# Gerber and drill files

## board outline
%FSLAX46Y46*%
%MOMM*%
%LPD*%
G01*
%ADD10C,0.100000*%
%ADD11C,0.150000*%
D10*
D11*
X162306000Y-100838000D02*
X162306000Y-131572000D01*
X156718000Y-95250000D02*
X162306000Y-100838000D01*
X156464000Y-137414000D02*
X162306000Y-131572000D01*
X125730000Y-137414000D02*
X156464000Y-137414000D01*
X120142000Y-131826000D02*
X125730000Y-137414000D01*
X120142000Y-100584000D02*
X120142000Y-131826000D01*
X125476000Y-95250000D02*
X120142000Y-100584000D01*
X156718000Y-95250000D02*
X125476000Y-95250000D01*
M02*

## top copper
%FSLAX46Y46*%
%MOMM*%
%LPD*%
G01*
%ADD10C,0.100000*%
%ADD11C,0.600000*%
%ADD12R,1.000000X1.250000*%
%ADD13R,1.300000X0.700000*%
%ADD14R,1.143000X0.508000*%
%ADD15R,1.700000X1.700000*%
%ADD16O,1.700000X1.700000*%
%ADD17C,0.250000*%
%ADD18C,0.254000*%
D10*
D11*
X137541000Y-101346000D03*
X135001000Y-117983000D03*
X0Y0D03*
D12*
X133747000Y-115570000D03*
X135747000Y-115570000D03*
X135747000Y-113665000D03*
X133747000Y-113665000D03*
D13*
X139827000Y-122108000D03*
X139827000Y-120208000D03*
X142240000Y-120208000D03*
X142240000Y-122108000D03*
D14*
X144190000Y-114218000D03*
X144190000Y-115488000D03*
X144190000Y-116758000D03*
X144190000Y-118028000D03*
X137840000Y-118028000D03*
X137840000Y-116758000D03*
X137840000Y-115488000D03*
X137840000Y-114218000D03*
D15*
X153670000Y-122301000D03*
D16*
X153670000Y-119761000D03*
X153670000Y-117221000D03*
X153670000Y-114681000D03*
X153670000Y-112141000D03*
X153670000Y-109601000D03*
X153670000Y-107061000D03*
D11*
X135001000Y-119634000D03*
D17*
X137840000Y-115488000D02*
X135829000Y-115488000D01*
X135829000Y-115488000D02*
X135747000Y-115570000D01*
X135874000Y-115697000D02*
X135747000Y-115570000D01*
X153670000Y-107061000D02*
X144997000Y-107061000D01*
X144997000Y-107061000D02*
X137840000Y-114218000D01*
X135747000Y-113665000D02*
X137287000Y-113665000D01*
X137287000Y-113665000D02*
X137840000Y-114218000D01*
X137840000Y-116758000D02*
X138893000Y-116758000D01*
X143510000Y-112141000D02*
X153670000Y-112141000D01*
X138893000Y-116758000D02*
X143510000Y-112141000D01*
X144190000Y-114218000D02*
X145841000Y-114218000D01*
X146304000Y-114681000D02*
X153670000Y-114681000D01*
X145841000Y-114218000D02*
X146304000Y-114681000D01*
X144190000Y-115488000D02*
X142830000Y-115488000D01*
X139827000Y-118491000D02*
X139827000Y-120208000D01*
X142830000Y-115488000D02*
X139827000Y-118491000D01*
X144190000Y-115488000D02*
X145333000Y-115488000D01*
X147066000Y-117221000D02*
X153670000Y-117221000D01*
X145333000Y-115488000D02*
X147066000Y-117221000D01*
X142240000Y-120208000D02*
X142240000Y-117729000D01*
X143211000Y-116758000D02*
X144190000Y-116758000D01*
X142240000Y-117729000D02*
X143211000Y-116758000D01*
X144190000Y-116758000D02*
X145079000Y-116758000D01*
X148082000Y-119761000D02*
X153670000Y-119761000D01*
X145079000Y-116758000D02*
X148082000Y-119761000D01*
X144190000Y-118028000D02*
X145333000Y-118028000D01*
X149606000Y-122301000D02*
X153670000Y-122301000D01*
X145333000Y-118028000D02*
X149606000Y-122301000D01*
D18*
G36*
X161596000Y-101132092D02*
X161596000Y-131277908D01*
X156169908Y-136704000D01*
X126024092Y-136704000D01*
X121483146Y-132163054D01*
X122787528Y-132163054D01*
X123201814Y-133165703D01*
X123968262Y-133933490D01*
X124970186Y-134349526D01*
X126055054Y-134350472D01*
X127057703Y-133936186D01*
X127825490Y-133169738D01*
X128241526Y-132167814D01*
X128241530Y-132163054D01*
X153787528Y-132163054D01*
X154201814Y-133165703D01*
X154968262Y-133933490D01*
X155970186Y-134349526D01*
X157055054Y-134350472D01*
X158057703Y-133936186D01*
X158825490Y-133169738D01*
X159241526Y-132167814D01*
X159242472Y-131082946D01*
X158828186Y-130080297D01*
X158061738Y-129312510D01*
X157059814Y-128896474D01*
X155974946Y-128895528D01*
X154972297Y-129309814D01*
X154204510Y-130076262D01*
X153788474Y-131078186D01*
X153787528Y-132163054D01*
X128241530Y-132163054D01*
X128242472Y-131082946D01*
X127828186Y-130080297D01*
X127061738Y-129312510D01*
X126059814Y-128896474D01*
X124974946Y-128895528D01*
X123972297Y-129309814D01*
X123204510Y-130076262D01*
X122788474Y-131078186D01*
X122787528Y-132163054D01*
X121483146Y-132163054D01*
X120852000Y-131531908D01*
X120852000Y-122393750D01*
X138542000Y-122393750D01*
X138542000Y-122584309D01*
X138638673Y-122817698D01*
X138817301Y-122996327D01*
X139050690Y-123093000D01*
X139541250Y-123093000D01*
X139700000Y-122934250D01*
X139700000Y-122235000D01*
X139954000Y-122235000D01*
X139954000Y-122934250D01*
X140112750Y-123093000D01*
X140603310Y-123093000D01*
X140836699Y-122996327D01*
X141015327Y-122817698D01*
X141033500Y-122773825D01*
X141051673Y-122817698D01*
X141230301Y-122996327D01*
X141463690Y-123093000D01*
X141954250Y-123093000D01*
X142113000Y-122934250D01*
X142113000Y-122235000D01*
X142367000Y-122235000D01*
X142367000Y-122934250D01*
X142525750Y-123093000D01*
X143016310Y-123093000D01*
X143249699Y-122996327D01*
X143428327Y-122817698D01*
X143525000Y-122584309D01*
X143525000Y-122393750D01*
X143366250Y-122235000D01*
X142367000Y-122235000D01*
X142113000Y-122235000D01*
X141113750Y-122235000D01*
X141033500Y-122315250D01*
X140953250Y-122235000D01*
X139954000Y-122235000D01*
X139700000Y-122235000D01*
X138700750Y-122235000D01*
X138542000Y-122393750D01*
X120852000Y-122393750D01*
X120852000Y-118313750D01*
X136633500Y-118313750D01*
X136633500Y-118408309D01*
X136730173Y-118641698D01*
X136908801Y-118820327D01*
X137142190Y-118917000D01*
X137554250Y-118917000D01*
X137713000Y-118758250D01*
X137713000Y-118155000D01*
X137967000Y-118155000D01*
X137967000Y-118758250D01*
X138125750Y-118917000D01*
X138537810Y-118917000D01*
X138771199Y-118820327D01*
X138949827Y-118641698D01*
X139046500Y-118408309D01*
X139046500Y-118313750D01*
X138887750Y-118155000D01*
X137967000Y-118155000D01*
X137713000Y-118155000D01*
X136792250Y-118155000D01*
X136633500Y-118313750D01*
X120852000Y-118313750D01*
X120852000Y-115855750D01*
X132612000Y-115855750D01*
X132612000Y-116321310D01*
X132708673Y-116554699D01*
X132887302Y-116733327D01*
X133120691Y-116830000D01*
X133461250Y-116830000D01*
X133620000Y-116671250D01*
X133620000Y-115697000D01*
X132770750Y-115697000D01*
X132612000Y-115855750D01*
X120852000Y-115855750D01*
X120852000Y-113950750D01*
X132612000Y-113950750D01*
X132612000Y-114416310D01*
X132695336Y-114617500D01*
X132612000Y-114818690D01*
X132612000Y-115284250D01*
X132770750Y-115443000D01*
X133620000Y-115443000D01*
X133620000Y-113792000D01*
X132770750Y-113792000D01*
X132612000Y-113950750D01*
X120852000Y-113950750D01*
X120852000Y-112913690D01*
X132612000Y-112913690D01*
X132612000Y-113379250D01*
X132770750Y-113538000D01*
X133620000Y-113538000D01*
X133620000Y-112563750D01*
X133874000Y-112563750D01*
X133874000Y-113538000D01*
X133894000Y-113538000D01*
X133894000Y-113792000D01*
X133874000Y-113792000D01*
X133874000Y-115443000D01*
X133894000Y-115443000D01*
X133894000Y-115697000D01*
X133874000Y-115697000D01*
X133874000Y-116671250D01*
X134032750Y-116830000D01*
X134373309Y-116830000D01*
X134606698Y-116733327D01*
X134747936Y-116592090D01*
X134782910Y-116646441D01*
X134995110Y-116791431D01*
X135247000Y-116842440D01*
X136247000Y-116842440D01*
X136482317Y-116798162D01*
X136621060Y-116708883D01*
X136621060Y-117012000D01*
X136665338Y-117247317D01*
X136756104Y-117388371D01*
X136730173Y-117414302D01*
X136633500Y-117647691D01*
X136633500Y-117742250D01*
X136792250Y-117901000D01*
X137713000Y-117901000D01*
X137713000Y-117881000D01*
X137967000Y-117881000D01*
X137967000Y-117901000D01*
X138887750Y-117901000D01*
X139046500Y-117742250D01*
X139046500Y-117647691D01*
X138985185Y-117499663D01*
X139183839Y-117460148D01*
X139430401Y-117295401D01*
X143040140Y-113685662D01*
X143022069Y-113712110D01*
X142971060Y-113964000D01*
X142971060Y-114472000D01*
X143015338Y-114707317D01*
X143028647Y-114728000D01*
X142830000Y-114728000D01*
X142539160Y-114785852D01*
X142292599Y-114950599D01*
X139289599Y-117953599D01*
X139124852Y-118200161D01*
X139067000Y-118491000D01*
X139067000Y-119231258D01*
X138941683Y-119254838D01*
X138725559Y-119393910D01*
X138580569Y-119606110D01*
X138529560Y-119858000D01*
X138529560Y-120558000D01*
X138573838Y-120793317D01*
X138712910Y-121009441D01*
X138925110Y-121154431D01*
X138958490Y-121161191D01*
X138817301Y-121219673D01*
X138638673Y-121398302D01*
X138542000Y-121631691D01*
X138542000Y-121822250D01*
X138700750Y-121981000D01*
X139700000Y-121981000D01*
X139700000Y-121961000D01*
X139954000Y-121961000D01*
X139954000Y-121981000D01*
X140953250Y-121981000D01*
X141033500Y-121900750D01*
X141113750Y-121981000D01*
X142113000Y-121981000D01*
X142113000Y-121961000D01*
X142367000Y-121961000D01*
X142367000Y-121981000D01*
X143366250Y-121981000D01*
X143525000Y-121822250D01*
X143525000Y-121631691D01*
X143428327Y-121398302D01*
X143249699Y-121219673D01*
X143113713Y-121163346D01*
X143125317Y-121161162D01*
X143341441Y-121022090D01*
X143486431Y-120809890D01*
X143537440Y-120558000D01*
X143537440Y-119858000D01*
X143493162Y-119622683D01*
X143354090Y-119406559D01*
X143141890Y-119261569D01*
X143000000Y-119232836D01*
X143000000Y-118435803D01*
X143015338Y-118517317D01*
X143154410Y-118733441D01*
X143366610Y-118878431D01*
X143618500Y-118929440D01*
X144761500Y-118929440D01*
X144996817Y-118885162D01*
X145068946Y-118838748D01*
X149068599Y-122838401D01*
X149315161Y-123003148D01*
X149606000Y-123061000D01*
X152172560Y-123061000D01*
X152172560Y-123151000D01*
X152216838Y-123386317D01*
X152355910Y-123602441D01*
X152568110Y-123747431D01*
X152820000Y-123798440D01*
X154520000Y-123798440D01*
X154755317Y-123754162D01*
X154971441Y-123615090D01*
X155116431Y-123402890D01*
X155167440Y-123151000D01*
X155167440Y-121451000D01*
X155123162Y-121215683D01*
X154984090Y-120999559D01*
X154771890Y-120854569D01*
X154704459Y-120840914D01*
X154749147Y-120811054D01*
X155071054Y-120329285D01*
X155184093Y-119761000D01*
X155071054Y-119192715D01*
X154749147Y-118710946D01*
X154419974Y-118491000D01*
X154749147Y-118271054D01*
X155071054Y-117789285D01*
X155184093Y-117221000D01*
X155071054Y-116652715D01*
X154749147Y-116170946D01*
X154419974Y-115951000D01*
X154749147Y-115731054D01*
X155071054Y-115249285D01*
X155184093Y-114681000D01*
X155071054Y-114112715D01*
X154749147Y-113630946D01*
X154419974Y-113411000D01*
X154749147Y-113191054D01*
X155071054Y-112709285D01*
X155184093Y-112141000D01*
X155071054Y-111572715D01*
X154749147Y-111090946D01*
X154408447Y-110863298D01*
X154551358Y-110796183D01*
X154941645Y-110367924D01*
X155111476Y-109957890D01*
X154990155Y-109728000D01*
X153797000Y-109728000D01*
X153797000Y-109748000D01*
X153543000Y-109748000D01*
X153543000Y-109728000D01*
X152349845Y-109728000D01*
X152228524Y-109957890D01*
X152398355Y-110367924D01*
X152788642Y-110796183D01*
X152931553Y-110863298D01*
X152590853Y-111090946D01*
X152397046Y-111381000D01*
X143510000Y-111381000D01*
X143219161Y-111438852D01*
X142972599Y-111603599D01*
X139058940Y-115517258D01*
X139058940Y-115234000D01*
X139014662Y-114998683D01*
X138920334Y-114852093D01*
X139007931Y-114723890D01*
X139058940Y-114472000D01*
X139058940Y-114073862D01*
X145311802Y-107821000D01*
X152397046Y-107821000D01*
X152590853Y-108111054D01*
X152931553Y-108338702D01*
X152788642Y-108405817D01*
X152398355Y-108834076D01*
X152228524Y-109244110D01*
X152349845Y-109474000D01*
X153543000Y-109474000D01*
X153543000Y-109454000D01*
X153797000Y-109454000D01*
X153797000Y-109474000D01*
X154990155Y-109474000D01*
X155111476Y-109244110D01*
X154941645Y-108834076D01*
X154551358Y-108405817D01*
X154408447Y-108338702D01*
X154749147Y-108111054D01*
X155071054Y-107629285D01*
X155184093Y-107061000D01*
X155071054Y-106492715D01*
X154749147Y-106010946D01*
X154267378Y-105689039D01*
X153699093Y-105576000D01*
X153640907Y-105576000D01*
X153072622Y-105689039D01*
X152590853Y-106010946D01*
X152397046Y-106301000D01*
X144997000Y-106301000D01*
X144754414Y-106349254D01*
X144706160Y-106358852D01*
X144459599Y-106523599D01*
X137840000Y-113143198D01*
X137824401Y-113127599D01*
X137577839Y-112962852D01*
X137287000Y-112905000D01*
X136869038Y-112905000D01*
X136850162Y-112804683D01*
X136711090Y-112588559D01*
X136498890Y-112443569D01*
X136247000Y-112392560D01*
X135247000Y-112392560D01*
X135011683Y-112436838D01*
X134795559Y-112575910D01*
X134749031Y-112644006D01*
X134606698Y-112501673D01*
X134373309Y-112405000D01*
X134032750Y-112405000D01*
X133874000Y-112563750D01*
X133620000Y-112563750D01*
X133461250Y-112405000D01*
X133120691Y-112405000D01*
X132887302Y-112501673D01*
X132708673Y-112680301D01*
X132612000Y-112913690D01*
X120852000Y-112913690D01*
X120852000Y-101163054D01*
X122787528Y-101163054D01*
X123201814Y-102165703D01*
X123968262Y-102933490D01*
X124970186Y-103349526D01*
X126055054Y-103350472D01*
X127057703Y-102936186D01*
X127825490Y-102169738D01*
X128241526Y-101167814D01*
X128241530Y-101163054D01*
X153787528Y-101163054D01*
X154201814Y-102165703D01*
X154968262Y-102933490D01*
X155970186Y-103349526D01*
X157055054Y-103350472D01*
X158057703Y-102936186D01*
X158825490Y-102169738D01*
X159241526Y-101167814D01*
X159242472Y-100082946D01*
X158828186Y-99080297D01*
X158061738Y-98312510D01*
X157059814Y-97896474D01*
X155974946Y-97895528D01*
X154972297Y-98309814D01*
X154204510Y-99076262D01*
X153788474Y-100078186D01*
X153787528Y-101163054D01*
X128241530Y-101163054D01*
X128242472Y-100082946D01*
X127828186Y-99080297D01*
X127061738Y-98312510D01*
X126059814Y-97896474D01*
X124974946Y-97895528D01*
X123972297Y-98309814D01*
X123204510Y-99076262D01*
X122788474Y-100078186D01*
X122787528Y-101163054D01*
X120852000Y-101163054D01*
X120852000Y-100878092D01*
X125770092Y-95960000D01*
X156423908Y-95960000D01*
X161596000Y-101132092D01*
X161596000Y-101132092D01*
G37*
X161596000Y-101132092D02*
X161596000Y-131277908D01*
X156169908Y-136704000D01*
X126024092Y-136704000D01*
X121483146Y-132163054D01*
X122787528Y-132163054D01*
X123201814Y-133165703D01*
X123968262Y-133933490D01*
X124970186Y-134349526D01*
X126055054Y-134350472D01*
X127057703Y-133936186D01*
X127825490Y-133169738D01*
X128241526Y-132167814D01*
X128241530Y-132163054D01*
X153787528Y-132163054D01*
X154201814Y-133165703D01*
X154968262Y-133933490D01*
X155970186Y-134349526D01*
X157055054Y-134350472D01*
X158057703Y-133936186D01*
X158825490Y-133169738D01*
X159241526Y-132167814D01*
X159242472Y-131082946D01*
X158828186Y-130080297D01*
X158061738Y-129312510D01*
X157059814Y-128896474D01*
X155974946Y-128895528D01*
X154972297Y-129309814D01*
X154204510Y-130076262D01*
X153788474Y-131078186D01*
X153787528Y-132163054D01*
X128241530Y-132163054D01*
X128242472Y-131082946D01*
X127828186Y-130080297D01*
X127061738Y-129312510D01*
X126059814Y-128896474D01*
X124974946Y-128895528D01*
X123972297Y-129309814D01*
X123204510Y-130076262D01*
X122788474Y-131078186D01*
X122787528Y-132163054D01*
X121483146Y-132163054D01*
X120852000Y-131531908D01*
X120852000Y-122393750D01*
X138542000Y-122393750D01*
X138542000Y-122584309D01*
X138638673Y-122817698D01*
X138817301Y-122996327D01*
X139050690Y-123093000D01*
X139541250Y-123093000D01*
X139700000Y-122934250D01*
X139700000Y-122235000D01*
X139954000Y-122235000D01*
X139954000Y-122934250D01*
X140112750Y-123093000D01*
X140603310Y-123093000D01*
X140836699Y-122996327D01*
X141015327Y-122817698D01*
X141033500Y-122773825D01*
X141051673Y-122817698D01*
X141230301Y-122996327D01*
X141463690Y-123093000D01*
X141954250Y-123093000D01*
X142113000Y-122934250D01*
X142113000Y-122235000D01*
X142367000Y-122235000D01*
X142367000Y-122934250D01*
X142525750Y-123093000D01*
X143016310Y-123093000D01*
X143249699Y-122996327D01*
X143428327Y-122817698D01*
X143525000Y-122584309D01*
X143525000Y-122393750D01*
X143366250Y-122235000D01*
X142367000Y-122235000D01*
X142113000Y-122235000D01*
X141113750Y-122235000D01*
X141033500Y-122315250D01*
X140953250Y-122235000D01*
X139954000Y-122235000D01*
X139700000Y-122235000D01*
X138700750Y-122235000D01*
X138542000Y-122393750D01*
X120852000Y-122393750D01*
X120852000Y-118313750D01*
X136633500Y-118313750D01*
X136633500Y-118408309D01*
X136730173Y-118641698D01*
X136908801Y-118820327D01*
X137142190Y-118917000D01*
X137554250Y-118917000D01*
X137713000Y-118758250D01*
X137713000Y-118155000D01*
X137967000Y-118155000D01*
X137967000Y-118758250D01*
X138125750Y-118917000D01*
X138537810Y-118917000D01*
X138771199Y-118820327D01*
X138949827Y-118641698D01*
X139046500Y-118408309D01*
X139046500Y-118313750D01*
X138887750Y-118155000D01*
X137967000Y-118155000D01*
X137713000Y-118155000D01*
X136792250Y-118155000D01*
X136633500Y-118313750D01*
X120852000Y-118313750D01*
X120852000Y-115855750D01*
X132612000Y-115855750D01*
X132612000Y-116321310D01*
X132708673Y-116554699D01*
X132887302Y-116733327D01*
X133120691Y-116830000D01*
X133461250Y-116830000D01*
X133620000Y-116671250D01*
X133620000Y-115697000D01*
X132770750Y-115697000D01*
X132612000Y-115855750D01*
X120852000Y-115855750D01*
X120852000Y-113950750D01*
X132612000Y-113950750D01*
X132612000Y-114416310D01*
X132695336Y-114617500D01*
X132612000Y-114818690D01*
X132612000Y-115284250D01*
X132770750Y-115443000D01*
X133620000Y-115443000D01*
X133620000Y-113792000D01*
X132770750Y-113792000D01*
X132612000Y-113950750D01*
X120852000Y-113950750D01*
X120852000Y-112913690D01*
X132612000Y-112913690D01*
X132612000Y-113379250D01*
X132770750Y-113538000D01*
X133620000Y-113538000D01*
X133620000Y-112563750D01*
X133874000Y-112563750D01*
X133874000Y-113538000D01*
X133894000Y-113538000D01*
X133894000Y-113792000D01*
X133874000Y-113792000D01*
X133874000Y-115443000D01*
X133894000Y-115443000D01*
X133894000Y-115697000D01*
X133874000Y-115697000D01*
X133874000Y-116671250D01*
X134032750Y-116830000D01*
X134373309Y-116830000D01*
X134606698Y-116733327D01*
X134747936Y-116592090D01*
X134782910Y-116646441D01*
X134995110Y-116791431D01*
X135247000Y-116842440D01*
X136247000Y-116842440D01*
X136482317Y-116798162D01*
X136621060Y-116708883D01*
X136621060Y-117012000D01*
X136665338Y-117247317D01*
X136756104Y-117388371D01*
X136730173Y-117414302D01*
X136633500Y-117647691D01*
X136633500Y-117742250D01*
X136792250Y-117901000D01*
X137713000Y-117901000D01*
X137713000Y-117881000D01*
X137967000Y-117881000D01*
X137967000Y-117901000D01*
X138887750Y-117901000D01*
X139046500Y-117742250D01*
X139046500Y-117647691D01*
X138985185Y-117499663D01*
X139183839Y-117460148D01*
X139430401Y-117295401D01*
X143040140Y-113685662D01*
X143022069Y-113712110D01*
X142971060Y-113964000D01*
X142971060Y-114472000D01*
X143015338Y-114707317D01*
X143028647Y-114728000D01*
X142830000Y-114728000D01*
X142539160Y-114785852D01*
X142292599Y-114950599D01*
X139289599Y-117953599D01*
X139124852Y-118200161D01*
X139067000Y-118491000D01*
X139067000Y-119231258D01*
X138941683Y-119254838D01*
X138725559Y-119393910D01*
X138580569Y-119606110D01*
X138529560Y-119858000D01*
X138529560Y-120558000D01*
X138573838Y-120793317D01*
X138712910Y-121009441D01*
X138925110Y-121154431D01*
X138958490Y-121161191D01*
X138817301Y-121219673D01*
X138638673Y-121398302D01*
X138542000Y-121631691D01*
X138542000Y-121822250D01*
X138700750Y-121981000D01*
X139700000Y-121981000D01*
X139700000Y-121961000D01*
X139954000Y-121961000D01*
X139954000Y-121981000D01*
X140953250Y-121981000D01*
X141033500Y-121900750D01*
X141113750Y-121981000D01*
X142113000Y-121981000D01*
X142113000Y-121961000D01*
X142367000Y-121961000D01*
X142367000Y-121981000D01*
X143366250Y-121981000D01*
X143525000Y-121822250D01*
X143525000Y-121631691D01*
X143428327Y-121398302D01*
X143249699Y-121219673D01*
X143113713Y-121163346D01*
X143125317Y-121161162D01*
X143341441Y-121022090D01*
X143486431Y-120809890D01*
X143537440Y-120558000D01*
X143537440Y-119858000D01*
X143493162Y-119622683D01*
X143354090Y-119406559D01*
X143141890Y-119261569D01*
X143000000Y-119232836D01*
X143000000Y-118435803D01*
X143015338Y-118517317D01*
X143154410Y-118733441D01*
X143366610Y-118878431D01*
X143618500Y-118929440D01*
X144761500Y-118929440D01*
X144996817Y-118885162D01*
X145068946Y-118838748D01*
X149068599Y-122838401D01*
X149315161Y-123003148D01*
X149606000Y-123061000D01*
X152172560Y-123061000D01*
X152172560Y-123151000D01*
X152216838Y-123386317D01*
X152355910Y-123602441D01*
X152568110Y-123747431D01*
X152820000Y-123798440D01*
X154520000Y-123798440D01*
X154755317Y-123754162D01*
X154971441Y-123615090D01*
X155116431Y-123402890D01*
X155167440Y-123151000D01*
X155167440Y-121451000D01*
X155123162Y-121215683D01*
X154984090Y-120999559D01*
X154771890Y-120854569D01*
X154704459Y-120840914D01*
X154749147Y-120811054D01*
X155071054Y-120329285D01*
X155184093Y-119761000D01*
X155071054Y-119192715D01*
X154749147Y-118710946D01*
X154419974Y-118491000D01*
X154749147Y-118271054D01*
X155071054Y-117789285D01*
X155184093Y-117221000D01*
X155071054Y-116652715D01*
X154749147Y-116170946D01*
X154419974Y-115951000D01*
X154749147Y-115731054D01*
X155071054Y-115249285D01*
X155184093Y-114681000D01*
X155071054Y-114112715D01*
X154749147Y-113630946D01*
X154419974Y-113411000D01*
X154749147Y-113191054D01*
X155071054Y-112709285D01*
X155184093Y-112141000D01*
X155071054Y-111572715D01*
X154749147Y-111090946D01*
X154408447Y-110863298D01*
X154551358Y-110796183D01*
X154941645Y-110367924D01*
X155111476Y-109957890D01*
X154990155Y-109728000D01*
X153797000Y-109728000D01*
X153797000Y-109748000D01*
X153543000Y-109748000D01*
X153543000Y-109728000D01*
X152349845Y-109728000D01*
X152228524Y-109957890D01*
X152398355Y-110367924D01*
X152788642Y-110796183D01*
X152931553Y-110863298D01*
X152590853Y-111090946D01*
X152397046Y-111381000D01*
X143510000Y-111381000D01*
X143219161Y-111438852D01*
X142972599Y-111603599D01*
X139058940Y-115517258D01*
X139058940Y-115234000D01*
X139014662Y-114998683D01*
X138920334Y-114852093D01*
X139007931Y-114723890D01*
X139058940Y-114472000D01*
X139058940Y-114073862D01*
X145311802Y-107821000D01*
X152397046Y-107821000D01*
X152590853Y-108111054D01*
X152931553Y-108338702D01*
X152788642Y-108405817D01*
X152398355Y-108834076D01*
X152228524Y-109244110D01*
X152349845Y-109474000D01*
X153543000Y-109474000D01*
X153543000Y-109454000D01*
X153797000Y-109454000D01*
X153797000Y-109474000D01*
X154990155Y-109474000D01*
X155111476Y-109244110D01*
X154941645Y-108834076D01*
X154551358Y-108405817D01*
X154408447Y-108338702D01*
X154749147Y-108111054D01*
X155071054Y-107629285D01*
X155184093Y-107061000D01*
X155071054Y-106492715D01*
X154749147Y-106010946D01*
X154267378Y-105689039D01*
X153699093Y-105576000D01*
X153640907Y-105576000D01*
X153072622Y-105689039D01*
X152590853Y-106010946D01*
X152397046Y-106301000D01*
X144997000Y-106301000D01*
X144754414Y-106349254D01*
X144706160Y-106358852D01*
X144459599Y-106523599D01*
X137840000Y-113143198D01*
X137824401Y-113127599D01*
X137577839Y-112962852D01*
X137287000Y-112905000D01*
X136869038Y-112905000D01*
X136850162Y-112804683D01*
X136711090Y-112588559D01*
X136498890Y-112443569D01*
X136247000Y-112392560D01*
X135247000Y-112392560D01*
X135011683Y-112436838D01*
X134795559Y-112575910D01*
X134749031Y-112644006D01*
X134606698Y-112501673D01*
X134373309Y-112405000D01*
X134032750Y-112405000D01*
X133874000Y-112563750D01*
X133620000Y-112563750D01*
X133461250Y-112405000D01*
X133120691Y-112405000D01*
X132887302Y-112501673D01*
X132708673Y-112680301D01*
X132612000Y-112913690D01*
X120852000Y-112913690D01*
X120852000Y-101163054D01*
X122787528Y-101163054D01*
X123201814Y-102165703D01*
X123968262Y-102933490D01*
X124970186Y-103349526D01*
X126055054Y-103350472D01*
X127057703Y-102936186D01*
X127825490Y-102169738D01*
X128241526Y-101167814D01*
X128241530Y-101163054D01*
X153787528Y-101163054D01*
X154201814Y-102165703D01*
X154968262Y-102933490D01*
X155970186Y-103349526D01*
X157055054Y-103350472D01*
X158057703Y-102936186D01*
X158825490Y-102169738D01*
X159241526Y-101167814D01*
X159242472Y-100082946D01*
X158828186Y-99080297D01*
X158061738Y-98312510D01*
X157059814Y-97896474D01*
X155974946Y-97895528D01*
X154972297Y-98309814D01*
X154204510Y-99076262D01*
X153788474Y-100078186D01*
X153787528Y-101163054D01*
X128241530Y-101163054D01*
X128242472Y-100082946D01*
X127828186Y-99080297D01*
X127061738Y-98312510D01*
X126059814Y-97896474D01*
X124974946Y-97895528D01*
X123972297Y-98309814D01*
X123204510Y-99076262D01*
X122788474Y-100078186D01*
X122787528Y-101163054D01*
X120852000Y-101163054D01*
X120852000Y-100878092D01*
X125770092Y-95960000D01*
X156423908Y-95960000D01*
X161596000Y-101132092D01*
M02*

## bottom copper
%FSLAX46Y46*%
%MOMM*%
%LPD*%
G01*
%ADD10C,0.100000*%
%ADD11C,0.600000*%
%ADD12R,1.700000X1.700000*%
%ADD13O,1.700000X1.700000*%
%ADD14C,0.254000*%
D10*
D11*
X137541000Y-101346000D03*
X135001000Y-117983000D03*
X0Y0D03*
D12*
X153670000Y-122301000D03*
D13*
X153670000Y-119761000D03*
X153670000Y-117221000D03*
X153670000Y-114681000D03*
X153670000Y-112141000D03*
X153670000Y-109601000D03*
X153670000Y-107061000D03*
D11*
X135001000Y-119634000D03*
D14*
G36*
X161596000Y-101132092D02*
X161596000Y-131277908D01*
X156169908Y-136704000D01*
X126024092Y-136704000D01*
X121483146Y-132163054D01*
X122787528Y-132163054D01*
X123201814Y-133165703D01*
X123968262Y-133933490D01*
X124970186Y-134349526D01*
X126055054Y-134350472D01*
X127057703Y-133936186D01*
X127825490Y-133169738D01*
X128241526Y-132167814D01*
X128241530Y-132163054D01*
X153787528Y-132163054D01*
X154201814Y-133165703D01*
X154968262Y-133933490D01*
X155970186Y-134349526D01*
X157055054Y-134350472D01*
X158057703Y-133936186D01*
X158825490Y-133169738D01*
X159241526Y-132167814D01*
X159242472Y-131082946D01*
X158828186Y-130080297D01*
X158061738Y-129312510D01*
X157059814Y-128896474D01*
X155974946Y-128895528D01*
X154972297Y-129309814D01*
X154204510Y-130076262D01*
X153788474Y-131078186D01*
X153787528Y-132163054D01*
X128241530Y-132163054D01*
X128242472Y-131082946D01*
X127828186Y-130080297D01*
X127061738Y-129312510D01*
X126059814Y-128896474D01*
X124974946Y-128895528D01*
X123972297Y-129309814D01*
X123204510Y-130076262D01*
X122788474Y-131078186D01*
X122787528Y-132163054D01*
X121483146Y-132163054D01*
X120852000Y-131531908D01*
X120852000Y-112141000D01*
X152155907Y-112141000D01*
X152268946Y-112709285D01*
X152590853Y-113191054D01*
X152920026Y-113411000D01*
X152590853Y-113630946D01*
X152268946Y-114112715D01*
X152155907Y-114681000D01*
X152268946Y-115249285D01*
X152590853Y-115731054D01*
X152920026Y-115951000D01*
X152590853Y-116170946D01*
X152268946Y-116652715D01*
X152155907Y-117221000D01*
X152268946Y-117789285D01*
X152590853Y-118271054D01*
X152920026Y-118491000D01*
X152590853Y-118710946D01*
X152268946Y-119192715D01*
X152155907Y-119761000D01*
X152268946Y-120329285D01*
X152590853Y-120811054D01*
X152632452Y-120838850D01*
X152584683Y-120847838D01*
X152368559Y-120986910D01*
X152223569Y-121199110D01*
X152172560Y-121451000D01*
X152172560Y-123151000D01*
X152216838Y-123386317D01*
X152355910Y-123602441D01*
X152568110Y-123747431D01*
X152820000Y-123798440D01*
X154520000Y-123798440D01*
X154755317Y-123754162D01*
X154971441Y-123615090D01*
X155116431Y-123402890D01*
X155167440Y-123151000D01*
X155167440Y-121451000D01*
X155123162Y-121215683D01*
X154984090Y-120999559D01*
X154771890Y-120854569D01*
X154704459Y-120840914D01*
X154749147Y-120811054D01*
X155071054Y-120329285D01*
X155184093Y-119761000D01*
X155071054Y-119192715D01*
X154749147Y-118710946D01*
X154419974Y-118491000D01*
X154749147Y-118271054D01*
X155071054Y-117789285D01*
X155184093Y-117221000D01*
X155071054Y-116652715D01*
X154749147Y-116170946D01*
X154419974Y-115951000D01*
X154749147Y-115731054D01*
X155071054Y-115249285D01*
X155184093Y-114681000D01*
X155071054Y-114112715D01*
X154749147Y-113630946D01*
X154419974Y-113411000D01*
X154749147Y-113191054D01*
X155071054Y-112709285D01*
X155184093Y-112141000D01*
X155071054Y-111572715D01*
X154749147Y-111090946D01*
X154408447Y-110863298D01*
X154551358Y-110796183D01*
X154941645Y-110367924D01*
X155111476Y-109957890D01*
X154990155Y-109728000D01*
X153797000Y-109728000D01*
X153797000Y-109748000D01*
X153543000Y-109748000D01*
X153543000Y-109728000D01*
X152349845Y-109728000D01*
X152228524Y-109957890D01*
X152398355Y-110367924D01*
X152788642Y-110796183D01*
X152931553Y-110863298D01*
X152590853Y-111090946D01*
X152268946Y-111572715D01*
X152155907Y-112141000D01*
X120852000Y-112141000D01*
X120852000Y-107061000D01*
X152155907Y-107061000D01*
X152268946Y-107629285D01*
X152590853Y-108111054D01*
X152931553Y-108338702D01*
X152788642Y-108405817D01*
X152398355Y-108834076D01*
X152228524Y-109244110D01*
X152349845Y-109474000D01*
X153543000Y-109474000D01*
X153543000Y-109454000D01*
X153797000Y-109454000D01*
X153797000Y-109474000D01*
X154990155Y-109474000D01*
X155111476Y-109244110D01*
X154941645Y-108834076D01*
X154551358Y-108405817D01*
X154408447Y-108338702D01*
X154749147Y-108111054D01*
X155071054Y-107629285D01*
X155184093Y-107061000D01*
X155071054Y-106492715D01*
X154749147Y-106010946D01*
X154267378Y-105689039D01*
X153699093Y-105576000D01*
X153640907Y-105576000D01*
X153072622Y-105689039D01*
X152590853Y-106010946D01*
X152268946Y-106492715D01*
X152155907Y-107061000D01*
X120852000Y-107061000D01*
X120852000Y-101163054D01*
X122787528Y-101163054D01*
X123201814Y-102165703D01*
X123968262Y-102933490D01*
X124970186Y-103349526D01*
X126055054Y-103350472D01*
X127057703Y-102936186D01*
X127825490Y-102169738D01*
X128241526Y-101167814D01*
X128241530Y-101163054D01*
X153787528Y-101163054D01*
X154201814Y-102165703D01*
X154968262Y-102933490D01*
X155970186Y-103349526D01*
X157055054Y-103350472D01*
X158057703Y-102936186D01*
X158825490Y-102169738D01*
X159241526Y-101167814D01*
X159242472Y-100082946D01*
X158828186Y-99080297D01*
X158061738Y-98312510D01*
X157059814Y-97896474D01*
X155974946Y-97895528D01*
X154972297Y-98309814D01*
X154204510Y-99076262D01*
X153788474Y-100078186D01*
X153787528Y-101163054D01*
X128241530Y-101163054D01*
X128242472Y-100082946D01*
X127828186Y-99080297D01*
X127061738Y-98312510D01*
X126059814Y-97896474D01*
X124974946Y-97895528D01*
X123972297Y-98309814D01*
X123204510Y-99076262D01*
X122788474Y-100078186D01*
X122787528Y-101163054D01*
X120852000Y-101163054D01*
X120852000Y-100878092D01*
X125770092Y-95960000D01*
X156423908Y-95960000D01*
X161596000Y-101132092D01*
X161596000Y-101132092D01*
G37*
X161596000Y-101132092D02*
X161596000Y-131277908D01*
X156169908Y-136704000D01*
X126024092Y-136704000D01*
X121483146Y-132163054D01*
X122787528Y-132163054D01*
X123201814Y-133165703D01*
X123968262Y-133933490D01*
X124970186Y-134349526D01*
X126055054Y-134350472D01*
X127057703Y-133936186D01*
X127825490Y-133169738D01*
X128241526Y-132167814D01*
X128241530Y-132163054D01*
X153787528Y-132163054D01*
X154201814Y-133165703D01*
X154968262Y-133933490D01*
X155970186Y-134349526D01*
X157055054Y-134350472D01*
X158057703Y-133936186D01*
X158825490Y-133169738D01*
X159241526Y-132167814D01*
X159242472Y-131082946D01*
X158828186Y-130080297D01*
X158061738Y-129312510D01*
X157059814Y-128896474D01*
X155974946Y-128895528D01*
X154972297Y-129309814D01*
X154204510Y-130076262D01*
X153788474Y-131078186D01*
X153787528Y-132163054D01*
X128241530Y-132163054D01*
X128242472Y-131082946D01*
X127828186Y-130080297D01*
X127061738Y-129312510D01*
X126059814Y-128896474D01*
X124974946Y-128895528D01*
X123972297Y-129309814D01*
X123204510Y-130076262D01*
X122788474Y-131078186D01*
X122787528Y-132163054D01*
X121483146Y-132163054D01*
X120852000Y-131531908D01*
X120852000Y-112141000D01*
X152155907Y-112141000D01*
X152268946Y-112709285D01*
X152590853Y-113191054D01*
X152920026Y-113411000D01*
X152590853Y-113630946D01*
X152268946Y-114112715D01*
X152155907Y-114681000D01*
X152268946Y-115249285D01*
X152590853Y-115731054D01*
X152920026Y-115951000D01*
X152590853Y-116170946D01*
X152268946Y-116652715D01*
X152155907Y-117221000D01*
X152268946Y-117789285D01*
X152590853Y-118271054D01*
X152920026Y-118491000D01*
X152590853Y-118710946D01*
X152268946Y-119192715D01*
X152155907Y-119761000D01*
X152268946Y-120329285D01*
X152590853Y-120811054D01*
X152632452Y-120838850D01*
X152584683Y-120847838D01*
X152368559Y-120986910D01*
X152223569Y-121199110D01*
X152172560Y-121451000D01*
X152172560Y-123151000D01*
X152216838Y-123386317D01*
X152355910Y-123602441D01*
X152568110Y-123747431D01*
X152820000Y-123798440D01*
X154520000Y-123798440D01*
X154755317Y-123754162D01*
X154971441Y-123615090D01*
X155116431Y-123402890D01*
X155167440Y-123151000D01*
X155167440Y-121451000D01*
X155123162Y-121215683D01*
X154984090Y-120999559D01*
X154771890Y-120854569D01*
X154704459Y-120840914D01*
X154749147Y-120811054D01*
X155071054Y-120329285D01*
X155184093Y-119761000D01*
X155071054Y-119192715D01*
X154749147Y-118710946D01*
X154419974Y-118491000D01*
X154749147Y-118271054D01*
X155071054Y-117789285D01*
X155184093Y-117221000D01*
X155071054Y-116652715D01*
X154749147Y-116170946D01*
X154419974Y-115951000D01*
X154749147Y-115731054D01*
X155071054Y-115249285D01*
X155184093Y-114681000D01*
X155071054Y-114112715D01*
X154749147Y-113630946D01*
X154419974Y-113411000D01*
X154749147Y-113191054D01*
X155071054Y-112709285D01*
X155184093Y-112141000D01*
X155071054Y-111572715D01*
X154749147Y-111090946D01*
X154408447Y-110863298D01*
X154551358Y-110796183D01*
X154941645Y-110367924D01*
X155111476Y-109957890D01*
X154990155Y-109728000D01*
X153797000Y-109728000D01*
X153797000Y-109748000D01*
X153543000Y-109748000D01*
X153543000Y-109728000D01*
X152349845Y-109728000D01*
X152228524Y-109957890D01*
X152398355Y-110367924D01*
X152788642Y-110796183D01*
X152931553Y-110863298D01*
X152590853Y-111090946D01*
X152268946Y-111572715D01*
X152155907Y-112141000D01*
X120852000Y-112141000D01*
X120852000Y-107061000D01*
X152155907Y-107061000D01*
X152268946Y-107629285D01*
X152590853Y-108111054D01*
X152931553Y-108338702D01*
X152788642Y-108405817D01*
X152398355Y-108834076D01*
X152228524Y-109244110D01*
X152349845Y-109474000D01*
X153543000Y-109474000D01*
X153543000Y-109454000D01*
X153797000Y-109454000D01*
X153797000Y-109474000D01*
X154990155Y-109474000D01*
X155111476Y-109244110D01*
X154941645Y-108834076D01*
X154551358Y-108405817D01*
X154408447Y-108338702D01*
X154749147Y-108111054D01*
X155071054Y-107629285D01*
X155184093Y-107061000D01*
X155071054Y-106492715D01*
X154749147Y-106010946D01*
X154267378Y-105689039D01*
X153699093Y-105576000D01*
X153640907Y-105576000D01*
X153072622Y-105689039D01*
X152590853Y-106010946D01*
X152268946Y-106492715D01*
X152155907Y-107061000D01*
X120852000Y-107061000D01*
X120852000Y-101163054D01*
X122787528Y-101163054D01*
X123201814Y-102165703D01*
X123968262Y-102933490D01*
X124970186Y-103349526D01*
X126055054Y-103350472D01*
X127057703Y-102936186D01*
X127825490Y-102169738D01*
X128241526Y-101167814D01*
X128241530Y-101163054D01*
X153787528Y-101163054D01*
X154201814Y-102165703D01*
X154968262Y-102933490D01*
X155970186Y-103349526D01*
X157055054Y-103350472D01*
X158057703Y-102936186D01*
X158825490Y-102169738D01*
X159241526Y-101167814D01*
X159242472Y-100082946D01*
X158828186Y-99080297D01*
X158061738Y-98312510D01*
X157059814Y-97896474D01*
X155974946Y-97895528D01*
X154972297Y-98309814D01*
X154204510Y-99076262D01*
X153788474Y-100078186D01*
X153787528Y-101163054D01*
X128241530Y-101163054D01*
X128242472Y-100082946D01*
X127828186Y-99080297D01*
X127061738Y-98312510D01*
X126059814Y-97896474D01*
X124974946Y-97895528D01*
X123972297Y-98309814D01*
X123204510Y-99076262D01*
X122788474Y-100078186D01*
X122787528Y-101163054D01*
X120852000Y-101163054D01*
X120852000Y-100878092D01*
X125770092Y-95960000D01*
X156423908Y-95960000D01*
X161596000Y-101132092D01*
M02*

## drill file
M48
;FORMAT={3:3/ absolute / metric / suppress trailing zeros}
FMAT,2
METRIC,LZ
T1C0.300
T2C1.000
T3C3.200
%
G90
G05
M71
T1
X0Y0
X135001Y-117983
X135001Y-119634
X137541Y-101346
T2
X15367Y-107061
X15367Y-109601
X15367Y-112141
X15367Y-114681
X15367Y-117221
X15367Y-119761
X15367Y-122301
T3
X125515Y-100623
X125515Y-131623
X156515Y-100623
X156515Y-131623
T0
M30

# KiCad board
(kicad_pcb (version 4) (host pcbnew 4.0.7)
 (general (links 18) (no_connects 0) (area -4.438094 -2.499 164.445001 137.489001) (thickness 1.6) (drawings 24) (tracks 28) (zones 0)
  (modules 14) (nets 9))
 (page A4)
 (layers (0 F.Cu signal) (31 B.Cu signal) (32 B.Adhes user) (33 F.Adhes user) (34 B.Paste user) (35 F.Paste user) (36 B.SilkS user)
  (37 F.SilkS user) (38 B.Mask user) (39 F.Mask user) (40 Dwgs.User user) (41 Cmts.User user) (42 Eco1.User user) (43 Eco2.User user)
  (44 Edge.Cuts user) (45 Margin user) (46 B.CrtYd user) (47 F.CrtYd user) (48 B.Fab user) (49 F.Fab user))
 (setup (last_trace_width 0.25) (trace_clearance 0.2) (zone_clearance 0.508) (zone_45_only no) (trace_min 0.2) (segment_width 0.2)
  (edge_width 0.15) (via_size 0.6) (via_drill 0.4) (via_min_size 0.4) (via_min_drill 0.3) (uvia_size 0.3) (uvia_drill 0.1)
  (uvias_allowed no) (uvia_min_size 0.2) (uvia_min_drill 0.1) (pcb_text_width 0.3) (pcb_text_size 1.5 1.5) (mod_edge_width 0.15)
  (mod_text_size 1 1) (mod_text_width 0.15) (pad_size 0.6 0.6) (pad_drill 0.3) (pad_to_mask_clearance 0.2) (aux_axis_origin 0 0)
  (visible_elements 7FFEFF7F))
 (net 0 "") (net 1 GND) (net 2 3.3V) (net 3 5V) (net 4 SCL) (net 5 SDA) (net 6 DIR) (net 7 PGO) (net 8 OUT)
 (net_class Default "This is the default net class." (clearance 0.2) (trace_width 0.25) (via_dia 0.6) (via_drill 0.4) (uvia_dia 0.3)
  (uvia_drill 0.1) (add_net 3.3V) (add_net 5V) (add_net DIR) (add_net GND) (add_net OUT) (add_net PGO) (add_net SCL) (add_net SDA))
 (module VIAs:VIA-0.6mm (layer F.Cu) (at 137.541 101.346)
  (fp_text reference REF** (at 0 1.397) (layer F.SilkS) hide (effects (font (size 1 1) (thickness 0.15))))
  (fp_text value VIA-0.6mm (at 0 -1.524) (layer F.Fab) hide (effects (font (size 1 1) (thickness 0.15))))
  (pad 1 thru_hole circle (at 0 0) (size 0.6 0.6) (drill 0.3) (layers *.Cu) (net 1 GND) (zone_connect 2)))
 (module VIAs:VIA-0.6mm (layer F.Cu) (at 135.001 117.983)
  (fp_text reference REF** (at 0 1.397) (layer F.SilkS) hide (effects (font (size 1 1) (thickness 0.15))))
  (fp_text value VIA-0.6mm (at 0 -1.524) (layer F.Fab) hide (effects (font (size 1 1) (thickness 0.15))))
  (pad 1 thru_hole circle (at 0 0) (size 0.6 0.6) (drill 0.3) (layers *.Cu) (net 1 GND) (zone_connect 2)))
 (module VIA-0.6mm (layer F.Cu) (at 0 0)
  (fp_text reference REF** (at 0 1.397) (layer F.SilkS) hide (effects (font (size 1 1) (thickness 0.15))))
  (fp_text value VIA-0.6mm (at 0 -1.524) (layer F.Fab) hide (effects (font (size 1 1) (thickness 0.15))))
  (pad 1 thru_hole circle (at 0 0) (size 0.6 0.6) (drill 0.3) (layers *.Cu) (zone_connect 2)))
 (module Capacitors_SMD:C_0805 (layer F.Cu) (at 134.747 115.57)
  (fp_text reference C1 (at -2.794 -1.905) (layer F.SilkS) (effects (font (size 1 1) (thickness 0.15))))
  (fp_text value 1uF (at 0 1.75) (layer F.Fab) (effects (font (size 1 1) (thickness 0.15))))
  (pad 1 smd rect (at -1 0) (size 1 1.25) (layers F.Cu F.Paste F.Mask) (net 1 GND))
  (pad 2 smd rect (at 1 0) (size 1 1.25) (layers F.Cu F.Paste F.Mask) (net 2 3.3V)))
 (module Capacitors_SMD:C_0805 (layer F.Cu) (at 134.747 113.665 180)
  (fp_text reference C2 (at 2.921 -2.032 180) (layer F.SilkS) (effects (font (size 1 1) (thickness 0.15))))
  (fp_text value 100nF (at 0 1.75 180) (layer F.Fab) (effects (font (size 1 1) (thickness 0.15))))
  (pad 1 smd rect (at -1 0 180) (size 1 1.25) (layers F.Cu F.Paste F.Mask) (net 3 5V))
  (pad 2 smd rect (at 1 0 180) (size 1 1.25) (layers F.Cu F.Paste F.Mask) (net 1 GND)))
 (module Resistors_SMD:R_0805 (layer F.Cu) (at 139.827 121.158 90)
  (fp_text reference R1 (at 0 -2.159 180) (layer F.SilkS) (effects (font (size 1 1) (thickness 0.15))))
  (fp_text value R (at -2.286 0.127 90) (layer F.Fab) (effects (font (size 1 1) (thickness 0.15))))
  (pad 1 smd rect (at -0.95 0 90) (size 0.7 1.3) (layers F.Cu F.Paste F.Mask) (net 1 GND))
  (pad 2 smd rect (at 0.95 0 90) (size 0.7 1.3) (layers F.Cu F.Paste F.Mask) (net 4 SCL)))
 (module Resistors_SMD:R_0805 (layer F.Cu) (at 142.24 121.158 270)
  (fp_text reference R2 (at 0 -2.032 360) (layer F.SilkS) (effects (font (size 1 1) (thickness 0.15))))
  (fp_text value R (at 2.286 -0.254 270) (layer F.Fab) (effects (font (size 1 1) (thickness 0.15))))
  (pad 1 smd rect (at -0.95 0 270) (size 0.7 1.3) (layers F.Cu F.Paste F.Mask) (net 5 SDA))
  (pad 2 smd rect (at 0.95 0 270) (size 0.7 1.3) (layers F.Cu F.Paste F.Mask) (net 1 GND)))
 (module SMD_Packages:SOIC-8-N (layer F.Cu) (at 141.015 116.123 270)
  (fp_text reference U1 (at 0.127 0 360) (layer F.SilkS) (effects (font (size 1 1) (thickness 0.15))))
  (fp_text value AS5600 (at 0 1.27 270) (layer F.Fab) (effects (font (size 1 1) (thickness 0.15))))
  (pad 8 smd rect (at -1.905 -3.175 270) (size 0.508 1.143) (layers F.Cu F.Paste F.Mask) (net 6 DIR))
  (pad 7 smd rect (at -0.635 -3.175 270) (size 0.508 1.143) (layers F.Cu F.Paste F.Mask) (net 4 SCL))
  (pad 6 smd rect (at 0.635 -3.175 270) (size 0.508 1.143) (layers F.Cu F.Paste F.Mask) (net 5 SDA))
  (pad 5 smd rect (at 1.905 -3.175 270) (size 0.508 1.143) (layers F.Cu F.Paste F.Mask) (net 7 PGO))
  (pad 4 smd rect (at 1.905 3.175 270) (size 0.508 1.143) (layers F.Cu F.Paste F.Mask) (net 1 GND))
  (pad 3 smd rect (at 0.635 3.175 270) (size 0.508 1.143) (layers F.Cu F.Paste F.Mask) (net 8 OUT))
  (pad 2 smd rect (at -0.635 3.175 270) (size 0.508 1.143) (layers F.Cu F.Paste F.Mask) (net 2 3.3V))
  (pad 1 smd rect (at -1.905 3.175 270) (size 0.508 1.143) (layers F.Cu F.Paste F.Mask) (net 3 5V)))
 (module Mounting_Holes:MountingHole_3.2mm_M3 (layer F.Cu) (at 125.515 100.623) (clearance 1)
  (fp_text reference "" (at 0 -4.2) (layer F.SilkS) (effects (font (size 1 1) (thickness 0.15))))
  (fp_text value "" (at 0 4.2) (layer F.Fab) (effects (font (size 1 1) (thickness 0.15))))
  (pad 1 np_thru_hole circle (at 0 0) (size 3.2 3.2) (drill 3.2) (layers *.Cu *.Mask)))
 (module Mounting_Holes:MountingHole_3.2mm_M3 (layer F.Cu) (at 156.515 100.623) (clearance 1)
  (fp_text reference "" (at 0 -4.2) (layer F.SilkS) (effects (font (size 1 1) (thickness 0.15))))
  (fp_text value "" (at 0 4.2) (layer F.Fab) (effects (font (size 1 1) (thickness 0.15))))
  (pad 1 np_thru_hole circle (at 0 0) (size 3.2 3.2) (drill 3.2) (layers *.Cu *.Mask)))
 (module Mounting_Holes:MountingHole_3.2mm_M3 (layer F.Cu) (at 125.515 131.623) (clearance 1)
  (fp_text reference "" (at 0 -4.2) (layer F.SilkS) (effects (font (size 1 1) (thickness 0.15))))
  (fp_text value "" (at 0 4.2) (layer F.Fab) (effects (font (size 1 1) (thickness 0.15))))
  (pad 1 np_thru_hole circle (at 0 0) (size 3.2 3.2) (drill 3.2) (layers *.Cu *.Mask)))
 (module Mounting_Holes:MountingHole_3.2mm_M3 (layer F.Cu) (at 156.515 131.623) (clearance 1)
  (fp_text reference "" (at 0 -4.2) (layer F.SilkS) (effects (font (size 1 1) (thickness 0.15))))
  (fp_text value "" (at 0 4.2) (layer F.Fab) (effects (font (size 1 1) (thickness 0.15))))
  (pad 1 np_thru_hole circle (at 0 0) (size 3.2 3.2) (drill 3.2) (layers *.Cu *.Mask)))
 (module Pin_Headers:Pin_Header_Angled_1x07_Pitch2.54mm (layer B.Cu) (at 153.67 122.301)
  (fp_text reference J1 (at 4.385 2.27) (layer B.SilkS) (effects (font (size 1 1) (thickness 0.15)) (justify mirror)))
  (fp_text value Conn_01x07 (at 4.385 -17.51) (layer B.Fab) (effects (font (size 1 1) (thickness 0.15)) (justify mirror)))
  (pad 1 thru_hole rect (at 0 0) (size 1.7 1.7) (drill 1) (layers *.Cu *.Mask) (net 7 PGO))
  (pad 2 thru_hole oval (at 0 -2.54) (size 1.7 1.7) (drill 1) (layers *.Cu *.Mask) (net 5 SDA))
  (pad 3 thru_hole oval (at 0 -5.08) (size 1.7 1.7) (drill 1) (layers *.Cu *.Mask) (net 4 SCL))
  (pad 4 thru_hole oval (at 0 -7.62) (size 1.7 1.7) (drill 1) (layers *.Cu *.Mask) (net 6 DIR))
  (pad 5 thru_hole oval (at 0 -10.16) (size 1.7 1.7) (drill 1) (layers *.Cu *.Mask) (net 8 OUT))
  (pad 6 thru_hole oval (at 0 -12.7) (size 1.7 1.7) (drill 1) (layers *.Cu *.Mask) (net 1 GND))
  (pad 7 thru_hole oval (at 0 -15.24) (size 1.7 1.7) (drill 1) (layers *.Cu *.Mask) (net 3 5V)))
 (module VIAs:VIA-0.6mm (layer F.Cu) (at 135.001 119.634)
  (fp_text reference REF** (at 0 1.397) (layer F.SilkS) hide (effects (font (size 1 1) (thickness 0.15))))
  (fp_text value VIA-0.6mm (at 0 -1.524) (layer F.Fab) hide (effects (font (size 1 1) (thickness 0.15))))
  (pad 1 thru_hole circle (at 0 0) (size 0.6 0.6) (drill 0.3) (layers *.Cu) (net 1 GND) (zone_connect 2)))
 (gr_line (start 162.306 100.838) (end 162.306 131.572) (angle 90) (layer Edge.Cuts) (width 0.15))
 (gr_line (start 156.718 95.25) (end 162.306 100.838) (angle 90) (layer Edge.Cuts) (width 0.15))
 (gr_line (start 156.464 137.414) (end 162.306 131.572) (angle 90) (layer Edge.Cuts) (width 0.15))
 (gr_line (start 125.73 137.414) (end 156.464 137.414) (angle 90) (layer Edge.Cuts) (width 0.15))
 (gr_line (start 120.142 131.826) (end 125.73 137.414) (angle 90) (layer Edge.Cuts) (width 0.15))
 (gr_line (start 120.142 100.584) (end 120.142 131.826) (angle 90) (layer Edge.Cuts) (width 0.15))
 (gr_line (start 125.476 95.25) (end 120.142 100.584) (angle 90) (layer Edge.Cuts) (width 0.15))
 (gr_line (start 156.718 95.25) (end 125.476 95.25) (angle 90) (layer Edge.Cuts) (width 0.15))
 (segment (start 137.84 115.488) (end 135.829 115.488) (width 0.25) (layer F.Cu) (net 2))
 (segment (start 135.829 115.488) (end 135.747 115.57) (width 0.25) (layer F.Cu) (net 2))
 (segment (start 135.874 115.697) (end 135.747 115.57) (width 0.25) (layer F.Cu) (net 2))
 (segment (start 153.67 107.061) (end 144.997 107.061) (width 0.25) (layer F.Cu) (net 3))
 (segment (start 144.997 107.061) (end 137.84 114.218) (width 0.25) (layer F.Cu) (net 3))
 (segment (start 135.747 113.665) (end 137.287 113.665) (width 0.25) (layer F.Cu) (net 3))
 (segment (start 137.287 113.665) (end 137.84 114.218) (width 0.25) (layer F.Cu) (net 3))
 (segment (start 137.84 116.758) (end 138.893 116.758) (width 0.25) (layer F.Cu) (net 8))
 (segment (start 143.51 112.141) (end 153.67 112.141) (width 0.25) (layer F.Cu) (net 8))
 (segment (start 138.893 116.758) (end 143.51 112.141) (width 0.25) (layer F.Cu) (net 8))
 (segment (start 144.19 114.218) (end 145.841 114.218) (width 0.25) (layer F.Cu) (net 6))
 (segment (start 146.304 114.681) (end 153.67 114.681) (width 0.25) (layer F.Cu) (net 6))
 (segment (start 145.841 114.218) (end 146.304 114.681) (width 0.25) (layer F.Cu) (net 6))
 (segment (start 144.19 115.488) (end 142.83 115.488) (width 0.25) (layer F.Cu) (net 4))
 (segment (start 139.827 118.491) (end 139.827 120.208) (width 0.25) (layer F.Cu) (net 4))
 (segment (start 142.83 115.488) (end 139.827 118.491) (width 0.25) (layer F.Cu) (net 4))
 (segment (start 144.19 115.488) (end 145.333 115.488) (width 0.25) (layer F.Cu) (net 4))
 (segment (start 147.066 117.221) (end 153.67 117.221) (width 0.25) (layer F.Cu) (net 4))
 (segment (start 145.333 115.488) (end 147.066 117.221) (width 0.25) (layer F.Cu) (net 4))
 (segment (start 142.24 120.208) (end 142.24 117.729) (width 0.25) (layer F.Cu) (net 5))
 (segment (start 143.211 116.758) (end 144.19 116.758) (width 0.25) (layer F.Cu) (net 5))
 (segment (start 142.24 117.729) (end 143.211 116.758) (width 0.25) (layer F.Cu) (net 5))
 (segment (start 144.19 116.758) (end 145.079 116.758) (width 0.25) (layer F.Cu) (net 5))
 (segment (start 148.082 119.761) (end 153.67 119.761) (width 0.25) (layer F.Cu) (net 5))
 (segment (start 145.079 116.758) (end 148.082 119.761) (width 0.25) (layer F.Cu) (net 5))
 (segment (start 144.19 118.028) (end 145.333 118.028) (width 0.25) (layer F.Cu) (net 7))
 (segment (start 149.606 122.301) (end 153.67 122.301) (width 0.25) (layer F.Cu) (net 7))
 (segment (start 145.333 118.028) (end 149.606 122.301) (width 0.25) (layer F.Cu) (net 7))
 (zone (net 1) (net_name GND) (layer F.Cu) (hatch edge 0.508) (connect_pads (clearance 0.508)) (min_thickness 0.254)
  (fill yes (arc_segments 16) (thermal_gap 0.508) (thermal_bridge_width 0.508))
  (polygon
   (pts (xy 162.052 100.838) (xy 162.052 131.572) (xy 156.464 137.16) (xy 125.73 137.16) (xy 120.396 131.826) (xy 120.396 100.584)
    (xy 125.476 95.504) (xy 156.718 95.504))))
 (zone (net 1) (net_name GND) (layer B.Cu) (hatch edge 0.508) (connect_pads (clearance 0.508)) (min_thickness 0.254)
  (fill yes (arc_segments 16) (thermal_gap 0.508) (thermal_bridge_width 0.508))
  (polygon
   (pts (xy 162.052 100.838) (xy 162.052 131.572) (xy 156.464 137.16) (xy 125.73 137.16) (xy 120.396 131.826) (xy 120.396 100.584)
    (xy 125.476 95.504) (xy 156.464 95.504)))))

